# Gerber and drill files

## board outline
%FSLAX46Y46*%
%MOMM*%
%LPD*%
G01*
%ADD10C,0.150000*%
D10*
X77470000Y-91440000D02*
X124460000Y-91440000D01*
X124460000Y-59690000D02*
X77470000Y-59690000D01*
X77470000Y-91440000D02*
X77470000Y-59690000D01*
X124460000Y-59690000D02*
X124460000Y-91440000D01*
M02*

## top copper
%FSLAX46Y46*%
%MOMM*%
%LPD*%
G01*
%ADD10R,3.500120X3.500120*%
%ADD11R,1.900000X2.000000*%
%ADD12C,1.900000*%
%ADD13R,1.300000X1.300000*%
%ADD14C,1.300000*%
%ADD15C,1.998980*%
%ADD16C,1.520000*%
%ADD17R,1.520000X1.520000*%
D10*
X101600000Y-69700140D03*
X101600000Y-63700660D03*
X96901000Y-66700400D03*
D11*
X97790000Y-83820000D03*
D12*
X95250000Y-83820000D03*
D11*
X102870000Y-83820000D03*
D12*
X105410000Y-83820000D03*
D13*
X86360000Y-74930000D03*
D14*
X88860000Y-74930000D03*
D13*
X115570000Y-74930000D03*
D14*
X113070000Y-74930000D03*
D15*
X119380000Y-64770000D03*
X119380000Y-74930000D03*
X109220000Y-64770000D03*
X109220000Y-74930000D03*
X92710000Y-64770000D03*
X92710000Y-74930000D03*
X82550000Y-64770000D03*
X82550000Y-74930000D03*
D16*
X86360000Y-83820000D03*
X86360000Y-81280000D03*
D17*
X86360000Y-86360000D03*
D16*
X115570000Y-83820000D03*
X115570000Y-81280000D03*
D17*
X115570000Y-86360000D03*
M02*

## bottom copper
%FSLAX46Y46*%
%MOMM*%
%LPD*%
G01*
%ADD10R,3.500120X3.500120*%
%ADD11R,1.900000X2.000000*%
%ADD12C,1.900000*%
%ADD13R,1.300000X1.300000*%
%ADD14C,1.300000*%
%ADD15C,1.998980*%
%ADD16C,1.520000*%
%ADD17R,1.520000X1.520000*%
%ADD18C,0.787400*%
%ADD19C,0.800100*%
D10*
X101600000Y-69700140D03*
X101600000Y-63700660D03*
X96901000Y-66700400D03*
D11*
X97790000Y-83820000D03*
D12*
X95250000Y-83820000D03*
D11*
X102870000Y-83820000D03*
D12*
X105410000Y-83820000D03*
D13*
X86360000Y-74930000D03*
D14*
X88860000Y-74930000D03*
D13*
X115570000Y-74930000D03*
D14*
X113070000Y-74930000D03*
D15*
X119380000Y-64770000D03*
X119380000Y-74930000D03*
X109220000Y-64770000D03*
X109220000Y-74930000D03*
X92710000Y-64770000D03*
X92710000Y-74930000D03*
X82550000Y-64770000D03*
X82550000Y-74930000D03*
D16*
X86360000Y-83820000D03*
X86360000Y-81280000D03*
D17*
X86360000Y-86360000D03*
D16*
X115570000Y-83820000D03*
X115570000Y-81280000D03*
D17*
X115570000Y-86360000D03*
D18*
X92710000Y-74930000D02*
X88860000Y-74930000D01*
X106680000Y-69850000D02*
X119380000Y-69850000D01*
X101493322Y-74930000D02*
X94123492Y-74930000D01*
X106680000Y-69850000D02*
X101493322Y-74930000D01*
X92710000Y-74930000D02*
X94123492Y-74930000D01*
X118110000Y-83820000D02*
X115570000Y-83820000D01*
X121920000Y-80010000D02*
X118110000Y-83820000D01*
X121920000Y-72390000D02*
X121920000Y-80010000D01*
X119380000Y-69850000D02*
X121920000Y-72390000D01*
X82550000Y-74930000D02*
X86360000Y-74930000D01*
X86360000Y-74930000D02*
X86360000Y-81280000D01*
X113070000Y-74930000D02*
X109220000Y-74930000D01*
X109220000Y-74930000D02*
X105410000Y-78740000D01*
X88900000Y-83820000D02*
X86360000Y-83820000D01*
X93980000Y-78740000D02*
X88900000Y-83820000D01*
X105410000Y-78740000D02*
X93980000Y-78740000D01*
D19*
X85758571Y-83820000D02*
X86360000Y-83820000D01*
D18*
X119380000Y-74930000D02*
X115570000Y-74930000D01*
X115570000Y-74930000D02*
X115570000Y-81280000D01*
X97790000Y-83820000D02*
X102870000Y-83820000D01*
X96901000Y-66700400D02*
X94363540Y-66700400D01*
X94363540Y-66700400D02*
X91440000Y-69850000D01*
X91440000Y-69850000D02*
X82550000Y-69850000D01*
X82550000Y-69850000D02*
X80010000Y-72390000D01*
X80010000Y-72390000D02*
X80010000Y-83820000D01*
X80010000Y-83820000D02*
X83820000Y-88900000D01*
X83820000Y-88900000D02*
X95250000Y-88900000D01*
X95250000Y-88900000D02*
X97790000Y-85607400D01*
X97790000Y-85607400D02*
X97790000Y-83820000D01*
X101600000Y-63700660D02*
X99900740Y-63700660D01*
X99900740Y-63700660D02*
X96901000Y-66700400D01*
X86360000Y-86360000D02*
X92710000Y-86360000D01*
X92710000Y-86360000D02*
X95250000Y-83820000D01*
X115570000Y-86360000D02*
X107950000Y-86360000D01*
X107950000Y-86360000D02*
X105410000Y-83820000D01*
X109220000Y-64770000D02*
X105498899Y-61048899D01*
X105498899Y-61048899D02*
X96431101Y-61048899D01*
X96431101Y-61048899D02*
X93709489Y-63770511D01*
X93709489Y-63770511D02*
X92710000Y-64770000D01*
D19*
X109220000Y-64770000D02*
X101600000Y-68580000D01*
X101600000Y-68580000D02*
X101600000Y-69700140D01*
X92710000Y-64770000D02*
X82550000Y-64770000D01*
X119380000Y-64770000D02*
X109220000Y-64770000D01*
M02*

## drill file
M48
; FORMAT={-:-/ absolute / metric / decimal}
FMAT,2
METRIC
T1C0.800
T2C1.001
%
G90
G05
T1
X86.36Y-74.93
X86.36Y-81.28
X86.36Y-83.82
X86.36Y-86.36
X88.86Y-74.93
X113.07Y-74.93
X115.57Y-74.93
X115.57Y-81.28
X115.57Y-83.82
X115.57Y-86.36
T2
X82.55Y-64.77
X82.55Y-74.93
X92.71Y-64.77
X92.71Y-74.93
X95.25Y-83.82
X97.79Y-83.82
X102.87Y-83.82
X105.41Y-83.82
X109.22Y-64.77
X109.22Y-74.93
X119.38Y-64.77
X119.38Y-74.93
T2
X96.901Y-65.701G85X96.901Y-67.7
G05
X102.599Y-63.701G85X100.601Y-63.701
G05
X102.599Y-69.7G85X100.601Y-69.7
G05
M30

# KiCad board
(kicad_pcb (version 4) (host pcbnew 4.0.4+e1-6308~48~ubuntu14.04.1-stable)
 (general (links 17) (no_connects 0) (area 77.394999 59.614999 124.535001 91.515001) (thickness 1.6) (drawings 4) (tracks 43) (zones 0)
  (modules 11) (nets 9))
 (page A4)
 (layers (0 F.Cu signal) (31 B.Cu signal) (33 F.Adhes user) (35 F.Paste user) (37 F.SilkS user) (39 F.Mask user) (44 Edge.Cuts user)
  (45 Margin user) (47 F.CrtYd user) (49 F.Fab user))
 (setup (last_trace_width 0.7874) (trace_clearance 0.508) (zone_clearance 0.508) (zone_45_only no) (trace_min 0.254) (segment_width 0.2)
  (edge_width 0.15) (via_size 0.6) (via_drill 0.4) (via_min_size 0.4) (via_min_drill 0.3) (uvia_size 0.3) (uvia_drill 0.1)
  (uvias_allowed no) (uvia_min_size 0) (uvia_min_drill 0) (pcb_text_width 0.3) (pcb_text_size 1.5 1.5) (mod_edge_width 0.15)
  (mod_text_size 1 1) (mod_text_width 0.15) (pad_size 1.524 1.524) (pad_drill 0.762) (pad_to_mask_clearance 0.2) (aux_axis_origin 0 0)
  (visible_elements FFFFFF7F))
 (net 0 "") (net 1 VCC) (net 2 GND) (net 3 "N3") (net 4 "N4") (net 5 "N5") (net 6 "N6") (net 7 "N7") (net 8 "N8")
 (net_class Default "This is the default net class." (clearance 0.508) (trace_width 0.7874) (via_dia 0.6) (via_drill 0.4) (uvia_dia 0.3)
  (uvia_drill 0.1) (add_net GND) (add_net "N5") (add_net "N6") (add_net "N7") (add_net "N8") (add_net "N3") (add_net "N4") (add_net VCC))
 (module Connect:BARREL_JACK (layer F.Cu) (at 101.6 63.5 270)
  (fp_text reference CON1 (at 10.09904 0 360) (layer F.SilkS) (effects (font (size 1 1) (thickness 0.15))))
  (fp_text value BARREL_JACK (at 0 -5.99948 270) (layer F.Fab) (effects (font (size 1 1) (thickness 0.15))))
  (pad 1 thru_hole rect (at 6.20014 0 270) (size 3.50012 3.50012) (drill oval 1.00076 2.99974) (layers *.Cu *.Mask F.SilkS) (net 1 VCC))
  (pad 2 thru_hole rect (at 0.20066 0 270) (size 3.50012 3.50012) (drill oval 1.00076 2.99974) (layers *.Cu *.Mask F.SilkS) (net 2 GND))
  (pad 3 thru_hole rect (at 3.2004 4.699 270) (size 3.50012 3.50012) (drill oval 2.99974 1.00076) (layers *.Cu *.Mask F.SilkS) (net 2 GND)))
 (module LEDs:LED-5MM (layer F.Cu) (at 97.79 83.82 180)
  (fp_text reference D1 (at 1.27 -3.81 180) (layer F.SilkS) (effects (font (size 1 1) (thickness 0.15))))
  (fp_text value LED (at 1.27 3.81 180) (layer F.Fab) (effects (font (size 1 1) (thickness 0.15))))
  (pad 1 thru_hole rect (at 0 0 270) (size 2 1.9) (drill 1.00076) (layers *.Cu *.Mask F.SilkS) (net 2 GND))
  (pad 2 thru_hole circle (at 2.54 0 180) (size 1.9 1.9) (drill 1.00076) (layers *.Cu *.Mask F.SilkS) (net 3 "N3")))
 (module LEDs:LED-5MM (layer F.Cu) (at 102.87 83.82)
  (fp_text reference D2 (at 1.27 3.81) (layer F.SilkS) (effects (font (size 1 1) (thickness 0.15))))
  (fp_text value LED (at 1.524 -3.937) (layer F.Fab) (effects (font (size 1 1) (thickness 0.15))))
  (pad 1 thru_hole rect (at 0 0 90) (size 2 1.9) (drill 1.00076) (layers *.Cu *.Mask F.SilkS) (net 2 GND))
  (pad 2 thru_hole circle (at 2.54 0) (size 1.9 1.9) (drill 1.00076) (layers *.Cu *.Mask F.SilkS) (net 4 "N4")))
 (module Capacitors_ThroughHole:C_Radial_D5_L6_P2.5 (layer F.Cu) (at 86.36 74.93)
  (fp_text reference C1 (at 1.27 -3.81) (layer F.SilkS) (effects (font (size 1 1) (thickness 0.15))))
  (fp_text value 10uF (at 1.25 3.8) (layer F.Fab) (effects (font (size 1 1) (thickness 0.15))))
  (pad 1 thru_hole rect (at 0 0) (size 1.3 1.3) (drill 0.8) (layers *.Cu *.Mask F.SilkS) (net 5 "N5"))
  (pad 2 thru_hole circle (at 2.5 0) (size 1.3 1.3) (drill 0.8) (layers *.Cu *.Mask F.SilkS) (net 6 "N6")))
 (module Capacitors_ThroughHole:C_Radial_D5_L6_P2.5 (layer F.Cu) (at 115.57 74.93 180)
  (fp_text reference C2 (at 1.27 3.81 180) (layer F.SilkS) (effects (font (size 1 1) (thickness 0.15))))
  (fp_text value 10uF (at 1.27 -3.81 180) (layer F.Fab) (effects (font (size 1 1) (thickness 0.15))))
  (pad 1 thru_hole rect (at 0 0 180) (size 1.3 1.3) (drill 0.8) (layers *.Cu *.Mask F.SilkS) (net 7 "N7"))
  (pad 2 thru_hole circle (at 2.5 0 180) (size 1.3 1.3) (drill 0.8) (layers *.Cu *.Mask F.SilkS) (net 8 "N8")))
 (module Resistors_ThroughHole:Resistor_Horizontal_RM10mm (layer F.Cu) (at 119.38 64.77 270)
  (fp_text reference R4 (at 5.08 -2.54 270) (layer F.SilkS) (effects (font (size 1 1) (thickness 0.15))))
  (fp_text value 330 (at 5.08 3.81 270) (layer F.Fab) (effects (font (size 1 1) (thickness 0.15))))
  (pad 1 thru_hole circle (at 0 0 270) (size 1.99898 1.99898) (drill 1.00076) (layers *.Cu *.SilkS *.Mask) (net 1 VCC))
  (pad 2 thru_hole circle (at 10.16 0 270) (size 1.99898 1.99898) (drill 1.00076) (layers *.Cu *.SilkS *.Mask) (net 7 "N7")))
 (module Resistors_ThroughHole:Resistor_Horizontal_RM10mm (layer F.Cu) (at 109.22 64.77 270)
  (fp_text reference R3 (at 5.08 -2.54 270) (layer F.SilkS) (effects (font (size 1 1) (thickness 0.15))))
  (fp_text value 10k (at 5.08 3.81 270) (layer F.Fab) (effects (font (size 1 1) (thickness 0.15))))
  (pad 1 thru_hole circle (at 0 0 270) (size 1.99898 1.99898) (drill 1.00076) (layers *.Cu *.SilkS *.Mask) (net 1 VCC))
  (pad 2 thru_hole circle (at 10.16 0 270) (size 1.99898 1.99898) (drill 1.00076) (layers *.Cu *.SilkS *.Mask) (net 8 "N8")))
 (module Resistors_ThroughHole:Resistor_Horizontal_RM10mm (layer F.Cu) (at 92.71 64.77 270)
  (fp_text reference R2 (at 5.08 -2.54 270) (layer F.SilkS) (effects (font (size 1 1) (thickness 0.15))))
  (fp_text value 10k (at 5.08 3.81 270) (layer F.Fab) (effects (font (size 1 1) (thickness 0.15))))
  (pad 1 thru_hole circle (at 0 0 270) (size 1.99898 1.99898) (drill 1.00076) (layers *.Cu *.SilkS *.Mask) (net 1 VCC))
  (pad 2 thru_hole circle (at 10.16 0 270) (size 1.99898 1.99898) (drill 1.00076) (layers *.Cu *.SilkS *.Mask) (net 6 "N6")))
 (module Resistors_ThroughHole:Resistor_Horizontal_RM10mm (layer F.Cu) (at 82.55 64.77 270)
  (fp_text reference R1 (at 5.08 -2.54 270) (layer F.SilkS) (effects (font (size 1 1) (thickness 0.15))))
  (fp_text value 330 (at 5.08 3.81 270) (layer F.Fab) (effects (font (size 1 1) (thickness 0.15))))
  (pad 1 thru_hole circle (at 0 0 270) (size 1.99898 1.99898) (drill 1.00076) (layers *.Cu *.SilkS *.Mask) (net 1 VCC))
  (pad 2 thru_hole circle (at 10.16 0 270) (size 1.99898 1.99898) (drill 1.00076) (layers *.Cu *.SilkS *.Mask) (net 5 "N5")))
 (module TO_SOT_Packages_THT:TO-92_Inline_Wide (layer F.Cu) (at 86.36 86.36 90)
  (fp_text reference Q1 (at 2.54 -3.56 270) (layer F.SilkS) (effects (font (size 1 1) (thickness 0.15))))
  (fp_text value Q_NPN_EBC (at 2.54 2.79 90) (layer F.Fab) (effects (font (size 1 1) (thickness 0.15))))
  (pad 2 thru_hole circle (at 2.54 0 180) (size 1.52 1.52) (drill 0.8) (layers *.Cu *.Mask) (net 8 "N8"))
  (pad 3 thru_hole circle (at 5.08 0 180) (size 1.52 1.52) (drill 0.8) (layers *.Cu *.Mask) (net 5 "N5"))
  (pad 1 thru_hole rect (at 0 0 180) (size 1.52 1.52) (drill 0.8) (layers *.Cu *.Mask) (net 3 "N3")))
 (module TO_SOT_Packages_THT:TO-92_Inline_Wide (layer F.Cu) (at 115.57 86.36 90)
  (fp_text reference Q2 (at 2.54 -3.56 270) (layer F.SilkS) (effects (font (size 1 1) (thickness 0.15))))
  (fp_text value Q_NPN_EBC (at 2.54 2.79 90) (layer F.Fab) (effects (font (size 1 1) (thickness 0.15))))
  (pad 2 thru_hole circle (at 2.54 0 180) (size 1.52 1.52) (drill 0.8) (layers *.Cu *.Mask) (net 6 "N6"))
  (pad 3 thru_hole circle (at 5.08 0 180) (size 1.52 1.52) (drill 0.8) (layers *.Cu *.Mask) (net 7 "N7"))
  (pad 1 thru_hole rect (at 0 0 180) (size 1.52 1.52) (drill 0.8) (layers *.Cu *.Mask) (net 4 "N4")))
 (gr_line (start 77.47 91.44) (end 124.46 91.44) (angle 90) (layer Edge.Cuts) (width 0.15))
 (gr_line (start 124.46 59.69) (end 77.47 59.69) (angle 90) (layer Edge.Cuts) (width 0.15))
 (gr_line (start 77.47 91.44) (end 77.47 59.69) (angle 90) (layer Edge.Cuts) (width 0.15))
 (gr_line (start 124.46 59.69) (end 124.46 91.44) (angle 90) (layer Edge.Cuts) (width 0.15))
 (segment (start 92.71 74.93) (end 88.86 74.93) (width 0.7874) (layer B.Cu) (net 6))
 (segment (start 106.68 69.85) (end 119.38 69.85) (width 0.7874) (layer B.Cu) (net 6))
 (segment (start 101.493322 74.93) (end 94.123492 74.93) (width 0.7874) (layer B.Cu) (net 6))
 (segment (start 106.68 69.85) (end 101.493322 74.93) (width 0.7874) (layer B.Cu) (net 6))
 (segment (start 92.71 74.93) (end 94.123492 74.93) (width 0.7874) (layer B.Cu) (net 6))
 (segment (start 118.11 83.82) (end 115.57 83.82) (width 0.7874) (layer B.Cu) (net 6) (status 20))
 (segment (start 121.92 80.01) (end 118.11 83.82) (width 0.7874) (layer B.Cu) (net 6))
 (segment (start 121.92 72.39) (end 121.92 80.01) (width 0.7874) (layer B.Cu) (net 6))
 (segment (start 119.38 69.85) (end 121.92 72.39) (width 0.7874) (layer B.Cu) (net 6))
 (segment (start 82.55 74.93) (end 86.36 74.93) (width 0.7874) (layer B.Cu) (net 5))
 (segment (start 86.36 74.93) (end 86.36 81.28) (width 0.7874) (layer B.Cu) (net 5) (status 10))
 (segment (start 113.07 74.93) (end 109.22 74.93) (width 0.7874) (layer B.Cu) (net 8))
 (segment (start 109.22 74.93) (end 105.41 78.74) (width 0.7874) (layer B.Cu) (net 8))
 (segment (start 88.9 83.82) (end 86.36 83.82) (width 0.7874) (layer B.Cu) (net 8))
 (segment (start 93.98 78.74) (end 88.9 83.82) (width 0.7874) (layer B.Cu) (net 8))
 (segment (start 105.41 78.74) (end 93.98 78.74) (width 0.7874) (layer B.Cu) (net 8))
 (segment (start 85.758571 83.82) (end 86.36 83.82) (width 0.8001) (layer B.Cu) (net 8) (status 30))
 (segment (start 119.38 74.93) (end 115.57 74.93) (width 0.7874) (layer B.Cu) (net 7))
 (segment (start 115.57 74.93) (end 115.57 81.28) (width 0.7874) (layer B.Cu) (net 7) (status 10))
 (segment (start 97.79 83.82) (end 102.87 83.82) (width 0.7874) (layer B.Cu) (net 2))
 (segment (start 96.901 66.7004) (end 94.36354 66.7004) (width 0.7874) (layer B.Cu) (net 2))
 (segment (start 94.36354 66.7004) (end 91.44 69.85) (width 0.7874) (layer B.Cu) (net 2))
 (segment (start 91.44 69.85) (end 82.55 69.85) (width 0.7874) (layer B.Cu) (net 2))
 (segment (start 82.55 69.85) (end 80.01 72.39) (width 0.7874) (layer B.Cu) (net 2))
 (segment (start 80.01 72.39) (end 80.01 83.82) (width 0.7874) (layer B.Cu) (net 2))
 (segment (start 80.01 83.82) (end 83.82 88.9) (width 0.7874) (layer B.Cu) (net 2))
 (segment (start 83.82 88.9) (end 95.25 88.9) (width 0.7874) (layer B.Cu) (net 2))
 (segment (start 95.25 88.9) (end 97.79 85.6074) (width 0.7874) (layer B.Cu) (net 2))
 (segment (start 97.79 85.6074) (end 97.79 83.82) (width 0.7874) (layer B.Cu) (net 2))
 (segment (start 101.6 63.70066) (end 99.90074 63.70066) (width 0.7874) (layer B.Cu) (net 2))
 (segment (start 99.90074 63.70066) (end 96.901 66.7004) (width 0.7874) (layer B.Cu) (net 2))
 (segment (start 86.36 86.36) (end 92.71 86.36) (width 0.7874) (layer B.Cu) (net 3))
 (segment (start 92.71 86.36) (end 95.25 83.82) (width 0.7874) (layer B.Cu) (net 3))
 (segment (start 115.57 86.36) (end 107.95 86.36) (width 0.7874) (layer B.Cu) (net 4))
 (segment (start 107.95 86.36) (end 105.41 83.82) (width 0.7874) (layer B.Cu) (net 4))
 (segment (start 109.22 64.77) (end 105.498899 61.048899) (width 0.7874) (layer B.Cu) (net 1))
 (segment (start 105.498899 61.048899) (end 96.431101 61.048899) (width 0.7874) (layer B.Cu) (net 1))
 (segment (start 96.431101 61.048899) (end 93.709489 63.770511) (width 0.7874) (layer B.Cu) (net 1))
 (segment (start 93.709489 63.770511) (end 92.71 64.77) (width 0.7874) (layer B.Cu) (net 1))
 (segment (start 109.22 64.77) (end 101.6 68.58) (width 0.8001) (layer B.Cu) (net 1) (status 30))
 (segment (start 101.6 68.58) (end 101.6 69.70014) (width 0.8001) (layer B.Cu) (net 1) (status 30))
 (segment (start 92.71 64.77) (end 82.55 64.77) (width 0.8001) (layer B.Cu) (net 1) (status 20))
 (segment (start 119.38 64.77) (end 109.22 64.77) (width 0.8001) (layer B.Cu) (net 1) (status 30)))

